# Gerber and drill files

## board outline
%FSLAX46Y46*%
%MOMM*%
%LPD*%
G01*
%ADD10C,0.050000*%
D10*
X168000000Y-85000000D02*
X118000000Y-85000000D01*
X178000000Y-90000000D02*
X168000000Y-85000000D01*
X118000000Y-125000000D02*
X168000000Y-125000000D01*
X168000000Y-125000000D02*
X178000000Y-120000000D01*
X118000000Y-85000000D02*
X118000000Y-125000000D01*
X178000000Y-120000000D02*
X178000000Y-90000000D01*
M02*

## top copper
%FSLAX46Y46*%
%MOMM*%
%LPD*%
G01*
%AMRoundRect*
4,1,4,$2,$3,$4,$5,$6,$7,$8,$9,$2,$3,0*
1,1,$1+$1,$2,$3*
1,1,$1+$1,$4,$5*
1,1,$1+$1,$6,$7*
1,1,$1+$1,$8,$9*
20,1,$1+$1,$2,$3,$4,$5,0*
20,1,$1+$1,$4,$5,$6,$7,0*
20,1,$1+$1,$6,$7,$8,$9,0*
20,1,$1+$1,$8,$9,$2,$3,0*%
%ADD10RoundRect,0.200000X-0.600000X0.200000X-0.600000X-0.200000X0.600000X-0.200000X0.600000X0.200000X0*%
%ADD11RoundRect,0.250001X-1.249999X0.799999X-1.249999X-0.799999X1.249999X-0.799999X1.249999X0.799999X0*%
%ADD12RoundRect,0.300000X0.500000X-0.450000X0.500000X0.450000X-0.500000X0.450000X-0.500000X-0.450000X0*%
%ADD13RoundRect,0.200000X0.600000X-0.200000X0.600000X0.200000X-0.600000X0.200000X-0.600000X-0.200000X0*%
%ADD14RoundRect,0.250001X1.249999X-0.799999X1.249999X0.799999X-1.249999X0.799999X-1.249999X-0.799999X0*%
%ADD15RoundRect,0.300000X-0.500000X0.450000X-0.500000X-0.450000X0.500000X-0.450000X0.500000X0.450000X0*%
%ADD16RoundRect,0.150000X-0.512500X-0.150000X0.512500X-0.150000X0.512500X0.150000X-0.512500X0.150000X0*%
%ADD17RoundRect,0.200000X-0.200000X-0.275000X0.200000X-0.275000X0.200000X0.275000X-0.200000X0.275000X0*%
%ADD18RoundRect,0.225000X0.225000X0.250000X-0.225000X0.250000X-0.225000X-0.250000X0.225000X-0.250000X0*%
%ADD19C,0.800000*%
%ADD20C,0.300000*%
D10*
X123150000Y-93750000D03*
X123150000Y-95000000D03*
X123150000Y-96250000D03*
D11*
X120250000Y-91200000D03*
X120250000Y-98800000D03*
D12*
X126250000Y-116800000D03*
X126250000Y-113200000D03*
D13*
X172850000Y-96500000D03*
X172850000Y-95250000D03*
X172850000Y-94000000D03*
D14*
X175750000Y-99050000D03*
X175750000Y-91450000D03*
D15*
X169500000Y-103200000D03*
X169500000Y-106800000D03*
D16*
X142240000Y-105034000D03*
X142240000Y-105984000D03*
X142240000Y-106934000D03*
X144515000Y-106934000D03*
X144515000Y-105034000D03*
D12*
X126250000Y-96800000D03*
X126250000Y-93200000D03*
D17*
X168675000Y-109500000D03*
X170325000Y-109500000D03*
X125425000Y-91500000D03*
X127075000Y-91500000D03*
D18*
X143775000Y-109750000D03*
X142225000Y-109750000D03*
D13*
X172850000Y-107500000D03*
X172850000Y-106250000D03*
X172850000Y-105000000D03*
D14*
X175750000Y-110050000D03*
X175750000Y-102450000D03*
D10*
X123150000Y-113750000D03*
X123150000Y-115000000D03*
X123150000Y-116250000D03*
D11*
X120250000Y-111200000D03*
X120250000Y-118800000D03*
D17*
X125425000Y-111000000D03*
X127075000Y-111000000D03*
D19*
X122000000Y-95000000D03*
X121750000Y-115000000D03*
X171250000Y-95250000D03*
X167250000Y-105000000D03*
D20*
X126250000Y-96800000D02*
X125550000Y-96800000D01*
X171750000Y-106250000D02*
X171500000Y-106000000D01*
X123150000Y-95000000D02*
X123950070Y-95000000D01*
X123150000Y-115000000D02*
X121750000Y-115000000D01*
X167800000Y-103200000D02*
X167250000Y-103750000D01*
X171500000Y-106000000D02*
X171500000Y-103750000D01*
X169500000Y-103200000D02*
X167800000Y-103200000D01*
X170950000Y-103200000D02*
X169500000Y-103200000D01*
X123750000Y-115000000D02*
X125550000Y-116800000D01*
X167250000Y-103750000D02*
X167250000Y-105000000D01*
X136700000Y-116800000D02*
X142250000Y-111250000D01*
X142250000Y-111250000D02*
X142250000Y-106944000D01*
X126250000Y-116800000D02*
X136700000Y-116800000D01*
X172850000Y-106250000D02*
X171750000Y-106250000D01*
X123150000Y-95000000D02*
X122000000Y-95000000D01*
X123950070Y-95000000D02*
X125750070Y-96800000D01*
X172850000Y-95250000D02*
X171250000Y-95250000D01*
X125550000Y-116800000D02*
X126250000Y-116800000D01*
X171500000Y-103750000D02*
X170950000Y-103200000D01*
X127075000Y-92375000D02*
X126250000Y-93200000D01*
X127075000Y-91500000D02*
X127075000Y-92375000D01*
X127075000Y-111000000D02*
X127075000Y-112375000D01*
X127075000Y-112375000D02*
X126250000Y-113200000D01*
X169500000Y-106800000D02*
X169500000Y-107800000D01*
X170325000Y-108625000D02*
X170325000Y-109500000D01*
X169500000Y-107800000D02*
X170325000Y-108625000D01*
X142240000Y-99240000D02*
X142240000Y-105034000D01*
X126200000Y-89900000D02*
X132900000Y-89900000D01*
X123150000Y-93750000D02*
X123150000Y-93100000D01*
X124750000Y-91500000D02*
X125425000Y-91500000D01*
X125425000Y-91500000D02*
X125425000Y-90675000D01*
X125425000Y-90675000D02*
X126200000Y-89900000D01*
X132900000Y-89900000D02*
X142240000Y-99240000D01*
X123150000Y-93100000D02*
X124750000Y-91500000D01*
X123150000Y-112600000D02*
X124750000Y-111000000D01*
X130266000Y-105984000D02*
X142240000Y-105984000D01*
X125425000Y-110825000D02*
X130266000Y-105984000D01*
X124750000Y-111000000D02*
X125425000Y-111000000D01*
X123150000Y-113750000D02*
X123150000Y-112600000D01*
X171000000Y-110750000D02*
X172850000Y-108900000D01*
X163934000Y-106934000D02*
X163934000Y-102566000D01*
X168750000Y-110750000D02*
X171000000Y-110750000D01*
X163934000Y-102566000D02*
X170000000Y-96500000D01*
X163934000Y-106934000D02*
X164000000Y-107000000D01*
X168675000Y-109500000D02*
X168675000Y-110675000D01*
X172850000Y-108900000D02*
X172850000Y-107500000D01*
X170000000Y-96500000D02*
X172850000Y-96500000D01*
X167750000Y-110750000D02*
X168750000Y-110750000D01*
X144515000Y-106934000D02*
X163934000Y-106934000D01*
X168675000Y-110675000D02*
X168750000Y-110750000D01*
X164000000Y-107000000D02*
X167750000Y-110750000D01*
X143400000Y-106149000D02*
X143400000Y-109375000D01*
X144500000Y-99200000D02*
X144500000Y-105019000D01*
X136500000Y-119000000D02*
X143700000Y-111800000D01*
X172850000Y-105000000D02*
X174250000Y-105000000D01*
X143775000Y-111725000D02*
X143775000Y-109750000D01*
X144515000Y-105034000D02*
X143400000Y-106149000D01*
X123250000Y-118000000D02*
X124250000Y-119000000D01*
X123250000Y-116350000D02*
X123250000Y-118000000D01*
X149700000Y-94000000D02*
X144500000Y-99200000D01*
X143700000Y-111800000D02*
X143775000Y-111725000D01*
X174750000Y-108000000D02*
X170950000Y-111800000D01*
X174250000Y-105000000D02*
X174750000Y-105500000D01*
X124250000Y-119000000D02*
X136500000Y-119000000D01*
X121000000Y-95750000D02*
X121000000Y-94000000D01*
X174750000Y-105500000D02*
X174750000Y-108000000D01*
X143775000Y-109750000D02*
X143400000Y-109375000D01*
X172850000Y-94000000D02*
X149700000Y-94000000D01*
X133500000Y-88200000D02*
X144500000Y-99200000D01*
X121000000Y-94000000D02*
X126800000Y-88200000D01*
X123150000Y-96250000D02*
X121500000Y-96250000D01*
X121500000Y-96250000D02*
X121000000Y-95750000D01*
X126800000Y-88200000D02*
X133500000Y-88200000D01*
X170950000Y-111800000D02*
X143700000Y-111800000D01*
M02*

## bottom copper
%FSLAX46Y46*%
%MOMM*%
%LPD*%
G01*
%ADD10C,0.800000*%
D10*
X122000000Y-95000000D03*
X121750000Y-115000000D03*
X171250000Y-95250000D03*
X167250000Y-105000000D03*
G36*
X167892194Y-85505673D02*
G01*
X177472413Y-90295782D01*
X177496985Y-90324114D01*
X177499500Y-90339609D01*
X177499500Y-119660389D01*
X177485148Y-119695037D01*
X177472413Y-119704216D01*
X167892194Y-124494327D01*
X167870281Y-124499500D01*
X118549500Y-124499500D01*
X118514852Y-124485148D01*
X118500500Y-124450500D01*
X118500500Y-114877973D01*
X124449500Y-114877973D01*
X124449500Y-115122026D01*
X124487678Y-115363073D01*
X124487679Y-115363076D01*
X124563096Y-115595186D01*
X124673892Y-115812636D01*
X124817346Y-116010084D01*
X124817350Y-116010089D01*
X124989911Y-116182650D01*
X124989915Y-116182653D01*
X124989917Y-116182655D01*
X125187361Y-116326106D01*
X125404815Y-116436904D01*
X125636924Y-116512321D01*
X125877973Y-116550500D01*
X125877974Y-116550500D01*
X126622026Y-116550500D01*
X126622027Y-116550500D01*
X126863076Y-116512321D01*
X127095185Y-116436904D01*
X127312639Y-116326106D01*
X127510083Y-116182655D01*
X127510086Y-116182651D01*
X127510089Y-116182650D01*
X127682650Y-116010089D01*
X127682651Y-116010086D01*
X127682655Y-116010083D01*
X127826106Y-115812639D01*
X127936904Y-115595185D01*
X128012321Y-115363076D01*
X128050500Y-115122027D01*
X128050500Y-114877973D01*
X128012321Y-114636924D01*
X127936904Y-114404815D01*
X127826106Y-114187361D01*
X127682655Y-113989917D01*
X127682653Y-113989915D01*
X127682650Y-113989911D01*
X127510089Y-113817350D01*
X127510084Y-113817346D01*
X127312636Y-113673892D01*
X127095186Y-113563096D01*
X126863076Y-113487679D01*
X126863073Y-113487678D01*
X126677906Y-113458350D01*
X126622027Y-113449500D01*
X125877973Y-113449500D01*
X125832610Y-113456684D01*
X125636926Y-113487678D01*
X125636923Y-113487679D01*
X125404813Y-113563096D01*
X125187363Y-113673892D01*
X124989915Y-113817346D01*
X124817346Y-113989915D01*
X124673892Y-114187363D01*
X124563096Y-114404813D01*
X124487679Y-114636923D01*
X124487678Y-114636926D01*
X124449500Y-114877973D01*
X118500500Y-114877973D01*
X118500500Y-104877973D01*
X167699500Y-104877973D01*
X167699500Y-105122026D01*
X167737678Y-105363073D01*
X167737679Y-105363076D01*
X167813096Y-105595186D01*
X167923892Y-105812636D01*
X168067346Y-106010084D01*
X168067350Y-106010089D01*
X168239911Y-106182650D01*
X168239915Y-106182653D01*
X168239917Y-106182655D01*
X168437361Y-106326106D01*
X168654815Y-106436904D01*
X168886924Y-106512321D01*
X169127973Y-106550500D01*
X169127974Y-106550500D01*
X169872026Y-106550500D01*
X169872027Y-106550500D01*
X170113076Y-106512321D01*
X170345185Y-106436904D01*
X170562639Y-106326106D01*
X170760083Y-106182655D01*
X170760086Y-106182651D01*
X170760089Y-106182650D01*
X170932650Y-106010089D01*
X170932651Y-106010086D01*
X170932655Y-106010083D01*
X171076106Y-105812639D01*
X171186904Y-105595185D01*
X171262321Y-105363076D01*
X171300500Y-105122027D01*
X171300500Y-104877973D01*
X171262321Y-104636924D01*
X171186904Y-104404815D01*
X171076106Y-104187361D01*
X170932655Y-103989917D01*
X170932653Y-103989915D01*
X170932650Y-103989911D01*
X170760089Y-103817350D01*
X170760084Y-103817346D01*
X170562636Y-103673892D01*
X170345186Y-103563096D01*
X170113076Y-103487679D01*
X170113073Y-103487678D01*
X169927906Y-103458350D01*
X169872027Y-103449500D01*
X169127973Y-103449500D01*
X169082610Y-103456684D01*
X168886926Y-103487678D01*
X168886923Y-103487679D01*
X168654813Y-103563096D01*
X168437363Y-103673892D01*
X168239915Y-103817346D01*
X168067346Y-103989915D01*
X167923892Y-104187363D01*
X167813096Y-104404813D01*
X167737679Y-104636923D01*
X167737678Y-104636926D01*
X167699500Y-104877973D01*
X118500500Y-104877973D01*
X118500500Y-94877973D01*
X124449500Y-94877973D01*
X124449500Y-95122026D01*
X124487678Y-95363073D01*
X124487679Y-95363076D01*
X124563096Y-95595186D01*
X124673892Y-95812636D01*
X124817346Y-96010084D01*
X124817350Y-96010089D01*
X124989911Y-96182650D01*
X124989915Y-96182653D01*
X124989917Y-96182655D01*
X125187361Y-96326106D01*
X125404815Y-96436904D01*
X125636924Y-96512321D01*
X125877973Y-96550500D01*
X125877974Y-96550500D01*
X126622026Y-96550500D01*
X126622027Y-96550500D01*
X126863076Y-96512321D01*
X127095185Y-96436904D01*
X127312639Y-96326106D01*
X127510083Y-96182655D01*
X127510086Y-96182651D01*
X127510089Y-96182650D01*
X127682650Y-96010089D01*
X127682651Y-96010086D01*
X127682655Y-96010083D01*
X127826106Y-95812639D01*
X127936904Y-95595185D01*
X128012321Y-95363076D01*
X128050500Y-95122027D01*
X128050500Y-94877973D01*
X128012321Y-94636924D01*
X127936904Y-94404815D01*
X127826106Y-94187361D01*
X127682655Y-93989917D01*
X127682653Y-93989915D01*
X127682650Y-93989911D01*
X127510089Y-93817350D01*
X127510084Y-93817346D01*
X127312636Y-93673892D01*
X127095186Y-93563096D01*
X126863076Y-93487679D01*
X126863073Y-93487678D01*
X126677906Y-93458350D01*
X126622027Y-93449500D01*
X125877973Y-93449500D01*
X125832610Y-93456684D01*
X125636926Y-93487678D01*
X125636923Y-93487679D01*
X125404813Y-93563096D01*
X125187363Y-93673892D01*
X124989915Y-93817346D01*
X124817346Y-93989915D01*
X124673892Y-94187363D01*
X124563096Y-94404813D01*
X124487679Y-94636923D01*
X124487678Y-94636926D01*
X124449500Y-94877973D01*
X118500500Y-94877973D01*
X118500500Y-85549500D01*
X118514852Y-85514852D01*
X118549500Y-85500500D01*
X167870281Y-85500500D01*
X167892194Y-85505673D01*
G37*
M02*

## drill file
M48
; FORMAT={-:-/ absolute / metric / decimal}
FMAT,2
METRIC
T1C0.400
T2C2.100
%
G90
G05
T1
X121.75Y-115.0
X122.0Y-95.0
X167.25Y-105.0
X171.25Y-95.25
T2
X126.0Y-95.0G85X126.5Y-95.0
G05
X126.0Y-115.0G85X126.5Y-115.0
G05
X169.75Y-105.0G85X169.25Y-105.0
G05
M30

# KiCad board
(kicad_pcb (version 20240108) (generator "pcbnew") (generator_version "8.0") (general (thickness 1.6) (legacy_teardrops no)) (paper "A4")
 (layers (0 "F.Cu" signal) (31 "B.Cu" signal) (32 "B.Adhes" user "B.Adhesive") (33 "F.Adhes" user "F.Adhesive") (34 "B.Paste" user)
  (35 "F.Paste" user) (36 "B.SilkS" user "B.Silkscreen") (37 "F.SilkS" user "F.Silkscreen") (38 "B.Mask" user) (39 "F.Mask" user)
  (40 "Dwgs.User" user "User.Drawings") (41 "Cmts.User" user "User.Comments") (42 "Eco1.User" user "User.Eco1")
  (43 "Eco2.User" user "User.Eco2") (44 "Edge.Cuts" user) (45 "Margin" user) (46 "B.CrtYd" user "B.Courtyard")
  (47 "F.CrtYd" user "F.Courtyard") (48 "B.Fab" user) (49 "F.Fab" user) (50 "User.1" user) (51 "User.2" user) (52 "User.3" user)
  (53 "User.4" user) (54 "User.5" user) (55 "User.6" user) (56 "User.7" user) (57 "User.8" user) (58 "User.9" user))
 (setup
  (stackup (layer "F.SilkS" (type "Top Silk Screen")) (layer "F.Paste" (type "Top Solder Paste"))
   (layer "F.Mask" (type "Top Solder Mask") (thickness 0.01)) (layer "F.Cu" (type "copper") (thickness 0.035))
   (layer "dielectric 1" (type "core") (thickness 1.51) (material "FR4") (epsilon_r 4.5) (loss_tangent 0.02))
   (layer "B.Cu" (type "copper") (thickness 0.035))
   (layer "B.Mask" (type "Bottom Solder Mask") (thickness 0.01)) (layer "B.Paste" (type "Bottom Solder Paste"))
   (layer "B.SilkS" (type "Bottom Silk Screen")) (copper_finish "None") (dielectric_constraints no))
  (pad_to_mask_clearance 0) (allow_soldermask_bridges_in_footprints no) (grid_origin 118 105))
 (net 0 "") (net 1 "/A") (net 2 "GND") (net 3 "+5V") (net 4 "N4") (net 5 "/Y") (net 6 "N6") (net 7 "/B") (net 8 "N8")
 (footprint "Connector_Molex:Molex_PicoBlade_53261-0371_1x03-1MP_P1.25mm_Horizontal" (layer "F.Cu") (at 120.75 95 -90)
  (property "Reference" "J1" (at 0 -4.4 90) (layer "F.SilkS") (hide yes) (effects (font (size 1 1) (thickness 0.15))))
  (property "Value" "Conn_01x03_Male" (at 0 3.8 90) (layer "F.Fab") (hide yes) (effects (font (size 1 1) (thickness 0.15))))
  (pad "1" smd roundrect (at -1.25 -2.4 270) (size 0.8 1.6) (layers "F.Cu" "F.Paste" "F.Mask") (roundrect_rratio 0.25) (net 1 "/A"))
  (pad "2" smd roundrect (at 0 -2.4 270) (size 0.8 1.6) (layers "F.Cu" "F.Paste" "F.Mask") (roundrect_rratio 0.25) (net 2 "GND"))
  (pad "3" smd roundrect (at 1.25 -2.4 270) (size 0.8 1.6) (layers "F.Cu" "F.Paste" "F.Mask") (roundrect_rratio 0.25) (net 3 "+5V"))
  (pad "MP" smd roundrect (at -3.8 0.5 270) (size 2.1 3) (layers "F.Cu" "F.Paste" "F.Mask") (roundrect_rratio 0.1190480952))
  (pad "MP" smd roundrect (at 3.8 0.5 270) (size 2.1 3) (layers "F.Cu" "F.Paste" "F.Mask") (roundrect_rratio 0.1190480952)))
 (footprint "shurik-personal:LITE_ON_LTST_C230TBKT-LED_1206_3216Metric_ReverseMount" (layer "F.Cu") (at 126.25 115 90)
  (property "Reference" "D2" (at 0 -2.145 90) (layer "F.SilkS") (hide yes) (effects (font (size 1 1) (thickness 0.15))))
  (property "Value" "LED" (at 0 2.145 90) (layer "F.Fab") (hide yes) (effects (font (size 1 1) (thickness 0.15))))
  (pad "" np_thru_hole oval (at 0 0 90) (size 2.1 2.6) (drill oval 2.1 2.6) (layers "F&B.Cu" "*.Mask"))
  (pad "1" smd roundrect (at -1.8 0 90) (size 1.5 1.6) (layers "F.Cu" "F.Paste" "F.Mask") (roundrect_rratio 0.2) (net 2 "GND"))
  (pad "2" smd roundrect (at 1.8 0 90) (size 1.5 1.6) (layers "F.Cu" "F.Paste" "F.Mask") (roundrect_rratio 0.2) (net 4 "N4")))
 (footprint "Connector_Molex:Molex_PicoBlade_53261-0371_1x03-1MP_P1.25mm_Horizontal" (layer "F.Cu") (at 175.25 95.25 90)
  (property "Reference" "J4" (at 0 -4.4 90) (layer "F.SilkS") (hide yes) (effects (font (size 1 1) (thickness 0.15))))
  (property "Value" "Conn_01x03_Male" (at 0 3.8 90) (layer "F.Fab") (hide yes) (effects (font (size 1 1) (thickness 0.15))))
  (pad "1" smd roundrect (at -1.25 -2.4 90) (size 0.8 1.6) (layers "F.Cu" "F.Paste" "F.Mask") (roundrect_rratio 0.25) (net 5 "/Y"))
  (pad "2" smd roundrect (at 0 -2.4 90) (size 0.8 1.6) (layers "F.Cu" "F.Paste" "F.Mask") (roundrect_rratio 0.25) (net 2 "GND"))
  (pad "3" smd roundrect (at 1.25 -2.4 90) (size 0.8 1.6) (layers "F.Cu" "F.Paste" "F.Mask") (roundrect_rratio 0.25) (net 3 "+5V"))
  (pad "MP" smd roundrect (at -3.8 0.5 90) (size 2.1 3) (layers "F.Cu" "F.Paste" "F.Mask") (roundrect_rratio 0.1190480952))
  (pad "MP" smd roundrect (at 3.8 0.5 90) (size 2.1 3) (layers "F.Cu" "F.Paste" "F.Mask") (roundrect_rratio 0.1190480952)))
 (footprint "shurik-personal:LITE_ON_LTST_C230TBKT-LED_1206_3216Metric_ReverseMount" (layer "F.Cu") (at 169.5 105 -90)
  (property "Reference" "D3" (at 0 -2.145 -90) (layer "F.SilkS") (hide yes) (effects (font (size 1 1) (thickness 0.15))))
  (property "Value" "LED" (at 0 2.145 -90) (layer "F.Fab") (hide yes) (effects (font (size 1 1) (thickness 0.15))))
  (pad "" np_thru_hole oval (at 0 0 270) (size 2.1 2.6) (drill oval 2.1 2.6) (layers "F&B.Cu" "*.Mask"))
  (pad "1" smd roundrect (at -1.8 0 270) (size 1.5 1.6) (layers "F.Cu" "F.Paste" "F.Mask") (roundrect_rratio 0.2) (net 2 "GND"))
  (pad "2" smd roundrect (at 1.8 0 270) (size 1.5 1.6) (layers "F.Cu" "F.Paste" "F.Mask") (roundrect_rratio 0.2) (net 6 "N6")))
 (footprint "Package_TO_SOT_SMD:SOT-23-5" (layer "F.Cu") (at 143.3775 105.984)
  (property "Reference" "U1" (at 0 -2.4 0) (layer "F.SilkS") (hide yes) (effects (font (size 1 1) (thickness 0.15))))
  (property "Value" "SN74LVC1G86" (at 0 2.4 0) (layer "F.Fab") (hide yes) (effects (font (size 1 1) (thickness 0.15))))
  (pad "1" smd roundrect (at -1.1375 -0.95) (size 1.325 0.6) (layers "F.Cu" "F.Paste" "F.Mask") (roundrect_rratio 0.25) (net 1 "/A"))
  (pad "2" smd roundrect (at -1.1375 0) (size 1.325 0.6) (layers "F.Cu" "F.Paste" "F.Mask") (roundrect_rratio 0.25) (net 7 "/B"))
  (pad "3" smd roundrect (at -1.1375 0.95) (size 1.325 0.6) (layers "F.Cu" "F.Paste" "F.Mask") (roundrect_rratio 0.25) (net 2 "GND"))
  (pad "4" smd roundrect (at 1.1375 0.95) (size 1.325 0.6) (layers "F.Cu" "F.Paste" "F.Mask") (roundrect_rratio 0.25) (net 5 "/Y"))
  (pad "5" smd roundrect (at 1.1375 -0.95) (size 1.325 0.6) (layers "F.Cu" "F.Paste" "F.Mask") (roundrect_rratio 0.25) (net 3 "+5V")))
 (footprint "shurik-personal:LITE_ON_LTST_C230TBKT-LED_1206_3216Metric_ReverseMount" (layer "F.Cu") (at 126.25 95 90)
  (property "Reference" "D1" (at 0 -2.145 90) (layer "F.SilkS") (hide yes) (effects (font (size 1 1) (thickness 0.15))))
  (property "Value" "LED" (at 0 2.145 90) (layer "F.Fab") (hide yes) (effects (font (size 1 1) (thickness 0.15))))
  (pad "" np_thru_hole oval (at 0 0 90) (size 2.1 2.6) (drill oval 2.1 2.6) (layers "F&B.Cu" "*.Mask"))
  (pad "1" smd roundrect (at -1.8 0 90) (size 1.5 1.6) (layers "F.Cu" "F.Paste" "F.Mask") (roundrect_rratio 0.2) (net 2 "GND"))
  (pad "2" smd roundrect (at 1.8 0 90) (size 1.5 1.6) (layers "F.Cu" "F.Paste" "F.Mask") (roundrect_rratio 0.2) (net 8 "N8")))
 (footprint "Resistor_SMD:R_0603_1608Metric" (layer "F.Cu") (at 169.5 109.5)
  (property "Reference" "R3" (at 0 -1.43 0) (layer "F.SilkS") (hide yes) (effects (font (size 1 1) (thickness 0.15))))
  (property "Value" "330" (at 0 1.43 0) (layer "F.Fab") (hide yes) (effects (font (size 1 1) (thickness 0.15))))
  (pad "1" smd roundrect (at -0.825 0) (size 0.8 0.95) (layers "F.Cu" "F.Paste" "F.Mask") (roundrect_rratio 0.25) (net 5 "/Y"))
  (pad "2" smd roundrect (at 0.825 0) (size 0.8 0.95) (layers "F.Cu" "F.Paste" "F.Mask") (roundrect_rratio 0.25) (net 6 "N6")))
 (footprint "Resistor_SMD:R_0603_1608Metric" (layer "F.Cu") (at 126.25 91.5)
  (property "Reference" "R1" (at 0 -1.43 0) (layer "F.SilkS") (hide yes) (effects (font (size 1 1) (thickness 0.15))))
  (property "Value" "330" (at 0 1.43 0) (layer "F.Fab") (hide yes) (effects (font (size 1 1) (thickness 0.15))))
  (pad "1" smd roundrect (at -0.825 0) (size 0.8 0.95) (layers "F.Cu" "F.Paste" "F.Mask") (roundrect_rratio 0.25) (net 1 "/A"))
  (pad "2" smd roundrect (at 0.825 0) (size 0.8 0.95) (layers "F.Cu" "F.Paste" "F.Mask") (roundrect_rratio 0.25) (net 8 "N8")))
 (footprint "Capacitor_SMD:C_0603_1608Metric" (layer "F.Cu") (at 143 109.75 180)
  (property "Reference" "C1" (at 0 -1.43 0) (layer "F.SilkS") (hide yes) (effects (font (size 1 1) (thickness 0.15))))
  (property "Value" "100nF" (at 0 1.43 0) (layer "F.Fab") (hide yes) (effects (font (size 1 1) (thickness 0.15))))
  (pad "1" smd roundrect (at -0.775 0 180) (size 0.9 0.95) (layers "F.Cu" "F.Paste" "F.Mask") (roundrect_rratio 0.25) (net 3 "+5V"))
  (pad "2" smd roundrect (at 0.775 0 180) (size 0.9 0.95) (layers "F.Cu" "F.Paste" "F.Mask") (roundrect_rratio 0.25) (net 2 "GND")))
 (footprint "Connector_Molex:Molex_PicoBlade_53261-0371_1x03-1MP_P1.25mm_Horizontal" (layer "F.Cu") (at 175.25 106.25 90)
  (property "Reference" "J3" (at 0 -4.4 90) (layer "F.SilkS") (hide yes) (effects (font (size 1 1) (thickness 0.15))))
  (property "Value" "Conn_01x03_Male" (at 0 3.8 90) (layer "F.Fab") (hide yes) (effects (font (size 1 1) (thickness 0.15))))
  (pad "1" smd roundrect (at -1.25 -2.4 90) (size 0.8 1.6) (layers "F.Cu" "F.Paste" "F.Mask") (roundrect_rratio 0.25) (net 5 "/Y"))
  (pad "2" smd roundrect (at 0 -2.4 90) (size 0.8 1.6) (layers "F.Cu" "F.Paste" "F.Mask") (roundrect_rratio 0.25) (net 2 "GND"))
  (pad "3" smd roundrect (at 1.25 -2.4 90) (size 0.8 1.6) (layers "F.Cu" "F.Paste" "F.Mask") (roundrect_rratio 0.25) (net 3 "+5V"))
  (pad "MP" smd roundrect (at -3.8 0.5 90) (size 2.1 3) (layers "F.Cu" "F.Paste" "F.Mask") (roundrect_rratio 0.1190480952))
  (pad "MP" smd roundrect (at 3.8 0.5 90) (size 2.1 3) (layers "F.Cu" "F.Paste" "F.Mask") (roundrect_rratio 0.1190480952)))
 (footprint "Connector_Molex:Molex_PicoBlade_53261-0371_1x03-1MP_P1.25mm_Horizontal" (layer "F.Cu") (at 120.75 115 -90)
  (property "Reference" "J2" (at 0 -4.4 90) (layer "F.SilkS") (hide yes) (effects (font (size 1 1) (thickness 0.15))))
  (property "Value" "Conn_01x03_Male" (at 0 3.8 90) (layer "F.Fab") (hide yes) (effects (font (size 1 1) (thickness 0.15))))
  (pad "1" smd roundrect (at -1.25 -2.4 270) (size 0.8 1.6) (layers "F.Cu" "F.Paste" "F.Mask") (roundrect_rratio 0.25) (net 7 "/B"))
  (pad "2" smd roundrect (at 0 -2.4 270) (size 0.8 1.6) (layers "F.Cu" "F.Paste" "F.Mask") (roundrect_rratio 0.25) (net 2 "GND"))
  (pad "3" smd roundrect (at 1.25 -2.4 270) (size 0.8 1.6) (layers "F.Cu" "F.Paste" "F.Mask") (roundrect_rratio 0.25) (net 3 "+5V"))
  (pad "MP" smd roundrect (at -3.8 0.5 270) (size 2.1 3) (layers "F.Cu" "F.Paste" "F.Mask") (roundrect_rratio 0.1190480952))
  (pad "MP" smd roundrect (at 3.8 0.5 270) (size 2.1 3) (layers "F.Cu" "F.Paste" "F.Mask") (roundrect_rratio 0.1190480952)))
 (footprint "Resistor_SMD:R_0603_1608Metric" (layer "F.Cu") (at 126.25 111)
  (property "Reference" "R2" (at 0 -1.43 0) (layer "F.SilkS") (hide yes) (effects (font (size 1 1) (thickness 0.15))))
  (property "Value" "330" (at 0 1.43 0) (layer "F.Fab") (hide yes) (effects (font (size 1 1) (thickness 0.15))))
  (pad "1" smd roundrect (at -0.825 0) (size 0.8 0.95) (layers "F.Cu" "F.Paste" "F.Mask") (roundrect_rratio 0.25) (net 7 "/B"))
  (pad "2" smd roundrect (at 0.825 0) (size 0.8 0.95) (layers "F.Cu" "F.Paste" "F.Mask") (roundrect_rratio 0.25) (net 4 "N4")))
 (gr_line (start 168 85) (end 118 85) (stroke (width 0.05) (type solid)) (layer "Edge.Cuts"))
 (gr_line (start 178 90) (end 168 85) (stroke (width 0.05) (type solid)) (layer "Edge.Cuts"))
 (gr_line (start 118 125) (end 168 125) (stroke (width 0.05) (type solid)) (layer "Edge.Cuts"))
 (gr_line (start 168 125) (end 178 120) (stroke (width 0.05) (type solid)) (layer "Edge.Cuts"))
 (gr_line (start 118 85) (end 118 125) (stroke (width 0.05) (type solid)) (layer "Edge.Cuts"))
 (gr_line (start 178 120) (end 178 90) (stroke (width 0.05) (type solid)) (layer "Edge.Cuts"))
 (segment (start 126.25 96.8) (end 125.55 96.8) (width 0.3) (layer "F.Cu") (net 2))
 (segment (start 171.75 106.25) (end 171.5 106) (width 0.3) (layer "F.Cu") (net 2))
 (segment (start 123.15 95) (end 123.95007 95) (width 0.3) (layer "F.Cu") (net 2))
 (segment (start 123.15 115) (end 121.75 115) (width 0.3) (layer "F.Cu") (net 2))
 (segment (start 167.8 103.2) (end 167.25 103.75) (width 0.3) (layer "F.Cu") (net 2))
 (segment (start 171.5 106) (end 171.5 103.75) (width 0.3) (layer "F.Cu") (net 2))
 (segment (start 169.5 103.2) (end 167.8 103.2) (width 0.3) (layer "F.Cu") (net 2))
 (segment (start 170.95 103.2) (end 169.5 103.2) (width 0.3) (layer "F.Cu") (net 2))
 (segment (start 123.75 115) (end 125.55 116.8) (width 0.3) (layer "F.Cu") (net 2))
 (segment (start 167.25 103.75) (end 167.25 105) (width 0.3) (layer "F.Cu") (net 2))
 (segment (start 136.7 116.8) (end 142.25 111.25) (width 0.3) (layer "F.Cu") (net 2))
 (segment (start 142.25 111.25) (end 142.25 106.944) (width 0.3) (layer "F.Cu") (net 2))
 (segment (start 126.25 116.8) (end 136.7 116.8) (width 0.3) (layer "F.Cu") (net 2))
 (segment (start 172.85 106.25) (end 171.75 106.25) (width 0.3) (layer "F.Cu") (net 2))
 (segment (start 123.15 95) (end 122 95) (width 0.3) (layer "F.Cu") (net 2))
 (segment (start 123.95007 95) (end 125.75007 96.8) (width 0.3) (layer "F.Cu") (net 2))
 (segment (start 172.85 95.25) (end 171.25 95.25) (width 0.3) (layer "F.Cu") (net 2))
 (segment (start 125.55 116.8) (end 126.25 116.8) (width 0.3) (layer "F.Cu") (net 2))
 (segment (start 171.5 103.75) (end 170.95 103.2) (width 0.3) (layer "F.Cu") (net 2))
 (via (at 122 95) (size 0.8) (drill 0.4) (layers "F.Cu" "B.Cu") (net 2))
 (via (at 121.75 115) (size 0.8) (drill 0.4) (layers "F.Cu" "B.Cu") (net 2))
 (via (at 171.25 95.25) (size 0.8) (drill 0.4) (layers "F.Cu" "B.Cu") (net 2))
 (via (at 167.25 105) (size 0.8) (drill 0.4) (layers "F.Cu" "B.Cu") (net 2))
 (segment (start 127.075 92.375) (end 126.25 93.2) (width 0.3) (layer "F.Cu") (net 8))
 (segment (start 127.075 91.5) (end 127.075 92.375) (width 0.3) (layer "F.Cu") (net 8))
 (segment (start 127.075 111) (end 127.075 112.375) (width 0.3) (layer "F.Cu") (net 4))
 (segment (start 127.075 112.375) (end 126.25 113.2) (width 0.3) (layer "F.Cu") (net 4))
 (segment (start 169.5 106.8) (end 169.5 107.8) (width 0.3) (layer "F.Cu") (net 6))
 (segment (start 170.325 108.625) (end 170.325 109.5) (width 0.3) (layer "F.Cu") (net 6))
 (segment (start 169.5 107.8) (end 170.325 108.625) (width 0.3) (layer "F.Cu") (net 6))
 (segment (start 142.24 99.24) (end 142.24 105.034) (width 0.3) (layer "F.Cu") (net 1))
 (segment (start 126.2 89.9) (end 132.9 89.9) (width 0.3) (layer "F.Cu") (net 1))
 (segment (start 123.15 93.75) (end 123.15 93.1) (width 0.3) (layer "F.Cu") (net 1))
 (segment (start 124.75 91.5) (end 125.425 91.5) (width 0.3) (layer "F.Cu") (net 1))
 (segment (start 125.425 91.5) (end 125.425 90.675) (width 0.3) (layer "F.Cu") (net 1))
 (segment (start 125.425 90.675) (end 126.2 89.9) (width 0.3) (layer "F.Cu") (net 1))
 (segment (start 132.9 89.9) (end 142.24 99.24) (width 0.3) (layer "F.Cu") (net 1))
 (segment (start 123.15 93.1) (end 124.75 91.5) (width 0.3) (layer "F.Cu") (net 1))
 (segment (start 123.15 112.6) (end 124.75 111) (width 0.3) (layer "F.Cu") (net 7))
 (segment (start 130.266 105.984) (end 142.24 105.984) (width 0.3) (layer "F.Cu") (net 7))
 (segment (start 125.425 110.825) (end 130.266 105.984) (width 0.3) (layer "F.Cu") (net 7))
 (segment (start 124.75 111) (end 125.425 111) (width 0.3) (layer "F.Cu") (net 7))
 (segment (start 123.15 113.75) (end 123.15 112.6) (width 0.3) (layer "F.Cu") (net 7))
 (segment (start 171 110.75) (end 172.85 108.9) (width 0.3) (layer "F.Cu") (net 5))
 (segment (start 163.934 106.934) (end 163.934 102.566) (width 0.3) (layer "F.Cu") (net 5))
 (segment (start 168.75 110.75) (end 171 110.75) (width 0.3) (layer "F.Cu") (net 5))
 (segment (start 163.934 102.566) (end 170 96.5) (width 0.3) (layer "F.Cu") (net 5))
 (segment (start 163.934 106.934) (end 164 107) (width 0.3) (layer "F.Cu") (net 5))
 (segment (start 168.675 109.5) (end 168.675 110.675) (width 0.3) (layer "F.Cu") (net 5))
 (segment (start 172.85 108.9) (end 172.85 107.5) (width 0.3) (layer "F.Cu") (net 5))
 (segment (start 170 96.5) (end 172.85 96.5) (width 0.3) (layer "F.Cu") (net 5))
 (segment (start 167.75 110.75) (end 168.75 110.75) (width 0.3) (layer "F.Cu") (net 5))
 (segment (start 144.515 106.934) (end 163.934 106.934) (width 0.3) (layer "F.Cu") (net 5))
 (segment (start 168.675 110.675) (end 168.75 110.75) (width 0.3) (layer "F.Cu") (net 5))
 (segment (start 164 107) (end 167.75 110.75) (width 0.3) (layer "F.Cu") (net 5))
 (segment (start 143.4 106.149) (end 143.4 109.375) (width 0.3) (layer "F.Cu") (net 3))
 (segment (start 144.5 99.2) (end 144.5 105.019) (width 0.3) (layer "F.Cu") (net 3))
 (segment (start 136.5 119) (end 143.7 111.8) (width 0.3) (layer "F.Cu") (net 3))
 (segment (start 172.85 105) (end 174.25 105) (width 0.3) (layer "F.Cu") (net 3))
 (segment (start 143.775 111.725) (end 143.775 109.75) (width 0.3) (layer "F.Cu") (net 3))
 (segment (start 144.515 105.034) (end 143.4 106.149) (width 0.3) (layer "F.Cu") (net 3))
 (segment (start 123.25 118) (end 124.25 119) (width 0.3) (layer "F.Cu") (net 3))
 (segment (start 123.25 116.35) (end 123.25 118) (width 0.3) (layer "F.Cu") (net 3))
 (segment (start 149.7 94) (end 144.5 99.2) (width 0.3) (layer "F.Cu") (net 3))
 (segment (start 143.7 111.8) (end 143.775 111.725) (width 0.3) (layer "F.Cu") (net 3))
 (segment (start 174.75 108) (end 170.95 111.8) (width 0.3) (layer "F.Cu") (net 3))
 (segment (start 174.25 105) (end 174.75 105.5) (width 0.3) (layer "F.Cu") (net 3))
 (segment (start 124.25 119) (end 136.5 119) (width 0.3) (layer "F.Cu") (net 3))
 (segment (start 121 95.75) (end 121 94) (width 0.3) (layer "F.Cu") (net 3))
 (segment (start 174.75 105.5) (end 174.75 108) (width 0.3) (layer "F.Cu") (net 3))
 (segment (start 143.775 109.75) (end 143.4 109.375) (width 0.3) (layer "F.Cu") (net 3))
 (segment (start 172.85 94) (end 149.7 94) (width 0.3) (layer "F.Cu") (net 3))
 (segment (start 133.5 88.2) (end 144.5 99.2) (width 0.3) (layer "F.Cu") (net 3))
 (segment (start 121 94) (end 126.8 88.2) (width 0.3) (layer "F.Cu") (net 3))
 (segment (start 123.15 96.25) (end 121.5 96.25) (width 0.3) (layer "F.Cu") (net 3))
 (segment (start 121.5 96.25) (end 121 95.75) (width 0.3) (layer "F.Cu") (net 3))
 (segment (start 126.8 88.2) (end 133.5 88.2) (width 0.3) (layer "F.Cu") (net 3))
 (segment (start 170.95 111.8) (end 143.7 111.8) (width 0.3) (layer "F.Cu") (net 3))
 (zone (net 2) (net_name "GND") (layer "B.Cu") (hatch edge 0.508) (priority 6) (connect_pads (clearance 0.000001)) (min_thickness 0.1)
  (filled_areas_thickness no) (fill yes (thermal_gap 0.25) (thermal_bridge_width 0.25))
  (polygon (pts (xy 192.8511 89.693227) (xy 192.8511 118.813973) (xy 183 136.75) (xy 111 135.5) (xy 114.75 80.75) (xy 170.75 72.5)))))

